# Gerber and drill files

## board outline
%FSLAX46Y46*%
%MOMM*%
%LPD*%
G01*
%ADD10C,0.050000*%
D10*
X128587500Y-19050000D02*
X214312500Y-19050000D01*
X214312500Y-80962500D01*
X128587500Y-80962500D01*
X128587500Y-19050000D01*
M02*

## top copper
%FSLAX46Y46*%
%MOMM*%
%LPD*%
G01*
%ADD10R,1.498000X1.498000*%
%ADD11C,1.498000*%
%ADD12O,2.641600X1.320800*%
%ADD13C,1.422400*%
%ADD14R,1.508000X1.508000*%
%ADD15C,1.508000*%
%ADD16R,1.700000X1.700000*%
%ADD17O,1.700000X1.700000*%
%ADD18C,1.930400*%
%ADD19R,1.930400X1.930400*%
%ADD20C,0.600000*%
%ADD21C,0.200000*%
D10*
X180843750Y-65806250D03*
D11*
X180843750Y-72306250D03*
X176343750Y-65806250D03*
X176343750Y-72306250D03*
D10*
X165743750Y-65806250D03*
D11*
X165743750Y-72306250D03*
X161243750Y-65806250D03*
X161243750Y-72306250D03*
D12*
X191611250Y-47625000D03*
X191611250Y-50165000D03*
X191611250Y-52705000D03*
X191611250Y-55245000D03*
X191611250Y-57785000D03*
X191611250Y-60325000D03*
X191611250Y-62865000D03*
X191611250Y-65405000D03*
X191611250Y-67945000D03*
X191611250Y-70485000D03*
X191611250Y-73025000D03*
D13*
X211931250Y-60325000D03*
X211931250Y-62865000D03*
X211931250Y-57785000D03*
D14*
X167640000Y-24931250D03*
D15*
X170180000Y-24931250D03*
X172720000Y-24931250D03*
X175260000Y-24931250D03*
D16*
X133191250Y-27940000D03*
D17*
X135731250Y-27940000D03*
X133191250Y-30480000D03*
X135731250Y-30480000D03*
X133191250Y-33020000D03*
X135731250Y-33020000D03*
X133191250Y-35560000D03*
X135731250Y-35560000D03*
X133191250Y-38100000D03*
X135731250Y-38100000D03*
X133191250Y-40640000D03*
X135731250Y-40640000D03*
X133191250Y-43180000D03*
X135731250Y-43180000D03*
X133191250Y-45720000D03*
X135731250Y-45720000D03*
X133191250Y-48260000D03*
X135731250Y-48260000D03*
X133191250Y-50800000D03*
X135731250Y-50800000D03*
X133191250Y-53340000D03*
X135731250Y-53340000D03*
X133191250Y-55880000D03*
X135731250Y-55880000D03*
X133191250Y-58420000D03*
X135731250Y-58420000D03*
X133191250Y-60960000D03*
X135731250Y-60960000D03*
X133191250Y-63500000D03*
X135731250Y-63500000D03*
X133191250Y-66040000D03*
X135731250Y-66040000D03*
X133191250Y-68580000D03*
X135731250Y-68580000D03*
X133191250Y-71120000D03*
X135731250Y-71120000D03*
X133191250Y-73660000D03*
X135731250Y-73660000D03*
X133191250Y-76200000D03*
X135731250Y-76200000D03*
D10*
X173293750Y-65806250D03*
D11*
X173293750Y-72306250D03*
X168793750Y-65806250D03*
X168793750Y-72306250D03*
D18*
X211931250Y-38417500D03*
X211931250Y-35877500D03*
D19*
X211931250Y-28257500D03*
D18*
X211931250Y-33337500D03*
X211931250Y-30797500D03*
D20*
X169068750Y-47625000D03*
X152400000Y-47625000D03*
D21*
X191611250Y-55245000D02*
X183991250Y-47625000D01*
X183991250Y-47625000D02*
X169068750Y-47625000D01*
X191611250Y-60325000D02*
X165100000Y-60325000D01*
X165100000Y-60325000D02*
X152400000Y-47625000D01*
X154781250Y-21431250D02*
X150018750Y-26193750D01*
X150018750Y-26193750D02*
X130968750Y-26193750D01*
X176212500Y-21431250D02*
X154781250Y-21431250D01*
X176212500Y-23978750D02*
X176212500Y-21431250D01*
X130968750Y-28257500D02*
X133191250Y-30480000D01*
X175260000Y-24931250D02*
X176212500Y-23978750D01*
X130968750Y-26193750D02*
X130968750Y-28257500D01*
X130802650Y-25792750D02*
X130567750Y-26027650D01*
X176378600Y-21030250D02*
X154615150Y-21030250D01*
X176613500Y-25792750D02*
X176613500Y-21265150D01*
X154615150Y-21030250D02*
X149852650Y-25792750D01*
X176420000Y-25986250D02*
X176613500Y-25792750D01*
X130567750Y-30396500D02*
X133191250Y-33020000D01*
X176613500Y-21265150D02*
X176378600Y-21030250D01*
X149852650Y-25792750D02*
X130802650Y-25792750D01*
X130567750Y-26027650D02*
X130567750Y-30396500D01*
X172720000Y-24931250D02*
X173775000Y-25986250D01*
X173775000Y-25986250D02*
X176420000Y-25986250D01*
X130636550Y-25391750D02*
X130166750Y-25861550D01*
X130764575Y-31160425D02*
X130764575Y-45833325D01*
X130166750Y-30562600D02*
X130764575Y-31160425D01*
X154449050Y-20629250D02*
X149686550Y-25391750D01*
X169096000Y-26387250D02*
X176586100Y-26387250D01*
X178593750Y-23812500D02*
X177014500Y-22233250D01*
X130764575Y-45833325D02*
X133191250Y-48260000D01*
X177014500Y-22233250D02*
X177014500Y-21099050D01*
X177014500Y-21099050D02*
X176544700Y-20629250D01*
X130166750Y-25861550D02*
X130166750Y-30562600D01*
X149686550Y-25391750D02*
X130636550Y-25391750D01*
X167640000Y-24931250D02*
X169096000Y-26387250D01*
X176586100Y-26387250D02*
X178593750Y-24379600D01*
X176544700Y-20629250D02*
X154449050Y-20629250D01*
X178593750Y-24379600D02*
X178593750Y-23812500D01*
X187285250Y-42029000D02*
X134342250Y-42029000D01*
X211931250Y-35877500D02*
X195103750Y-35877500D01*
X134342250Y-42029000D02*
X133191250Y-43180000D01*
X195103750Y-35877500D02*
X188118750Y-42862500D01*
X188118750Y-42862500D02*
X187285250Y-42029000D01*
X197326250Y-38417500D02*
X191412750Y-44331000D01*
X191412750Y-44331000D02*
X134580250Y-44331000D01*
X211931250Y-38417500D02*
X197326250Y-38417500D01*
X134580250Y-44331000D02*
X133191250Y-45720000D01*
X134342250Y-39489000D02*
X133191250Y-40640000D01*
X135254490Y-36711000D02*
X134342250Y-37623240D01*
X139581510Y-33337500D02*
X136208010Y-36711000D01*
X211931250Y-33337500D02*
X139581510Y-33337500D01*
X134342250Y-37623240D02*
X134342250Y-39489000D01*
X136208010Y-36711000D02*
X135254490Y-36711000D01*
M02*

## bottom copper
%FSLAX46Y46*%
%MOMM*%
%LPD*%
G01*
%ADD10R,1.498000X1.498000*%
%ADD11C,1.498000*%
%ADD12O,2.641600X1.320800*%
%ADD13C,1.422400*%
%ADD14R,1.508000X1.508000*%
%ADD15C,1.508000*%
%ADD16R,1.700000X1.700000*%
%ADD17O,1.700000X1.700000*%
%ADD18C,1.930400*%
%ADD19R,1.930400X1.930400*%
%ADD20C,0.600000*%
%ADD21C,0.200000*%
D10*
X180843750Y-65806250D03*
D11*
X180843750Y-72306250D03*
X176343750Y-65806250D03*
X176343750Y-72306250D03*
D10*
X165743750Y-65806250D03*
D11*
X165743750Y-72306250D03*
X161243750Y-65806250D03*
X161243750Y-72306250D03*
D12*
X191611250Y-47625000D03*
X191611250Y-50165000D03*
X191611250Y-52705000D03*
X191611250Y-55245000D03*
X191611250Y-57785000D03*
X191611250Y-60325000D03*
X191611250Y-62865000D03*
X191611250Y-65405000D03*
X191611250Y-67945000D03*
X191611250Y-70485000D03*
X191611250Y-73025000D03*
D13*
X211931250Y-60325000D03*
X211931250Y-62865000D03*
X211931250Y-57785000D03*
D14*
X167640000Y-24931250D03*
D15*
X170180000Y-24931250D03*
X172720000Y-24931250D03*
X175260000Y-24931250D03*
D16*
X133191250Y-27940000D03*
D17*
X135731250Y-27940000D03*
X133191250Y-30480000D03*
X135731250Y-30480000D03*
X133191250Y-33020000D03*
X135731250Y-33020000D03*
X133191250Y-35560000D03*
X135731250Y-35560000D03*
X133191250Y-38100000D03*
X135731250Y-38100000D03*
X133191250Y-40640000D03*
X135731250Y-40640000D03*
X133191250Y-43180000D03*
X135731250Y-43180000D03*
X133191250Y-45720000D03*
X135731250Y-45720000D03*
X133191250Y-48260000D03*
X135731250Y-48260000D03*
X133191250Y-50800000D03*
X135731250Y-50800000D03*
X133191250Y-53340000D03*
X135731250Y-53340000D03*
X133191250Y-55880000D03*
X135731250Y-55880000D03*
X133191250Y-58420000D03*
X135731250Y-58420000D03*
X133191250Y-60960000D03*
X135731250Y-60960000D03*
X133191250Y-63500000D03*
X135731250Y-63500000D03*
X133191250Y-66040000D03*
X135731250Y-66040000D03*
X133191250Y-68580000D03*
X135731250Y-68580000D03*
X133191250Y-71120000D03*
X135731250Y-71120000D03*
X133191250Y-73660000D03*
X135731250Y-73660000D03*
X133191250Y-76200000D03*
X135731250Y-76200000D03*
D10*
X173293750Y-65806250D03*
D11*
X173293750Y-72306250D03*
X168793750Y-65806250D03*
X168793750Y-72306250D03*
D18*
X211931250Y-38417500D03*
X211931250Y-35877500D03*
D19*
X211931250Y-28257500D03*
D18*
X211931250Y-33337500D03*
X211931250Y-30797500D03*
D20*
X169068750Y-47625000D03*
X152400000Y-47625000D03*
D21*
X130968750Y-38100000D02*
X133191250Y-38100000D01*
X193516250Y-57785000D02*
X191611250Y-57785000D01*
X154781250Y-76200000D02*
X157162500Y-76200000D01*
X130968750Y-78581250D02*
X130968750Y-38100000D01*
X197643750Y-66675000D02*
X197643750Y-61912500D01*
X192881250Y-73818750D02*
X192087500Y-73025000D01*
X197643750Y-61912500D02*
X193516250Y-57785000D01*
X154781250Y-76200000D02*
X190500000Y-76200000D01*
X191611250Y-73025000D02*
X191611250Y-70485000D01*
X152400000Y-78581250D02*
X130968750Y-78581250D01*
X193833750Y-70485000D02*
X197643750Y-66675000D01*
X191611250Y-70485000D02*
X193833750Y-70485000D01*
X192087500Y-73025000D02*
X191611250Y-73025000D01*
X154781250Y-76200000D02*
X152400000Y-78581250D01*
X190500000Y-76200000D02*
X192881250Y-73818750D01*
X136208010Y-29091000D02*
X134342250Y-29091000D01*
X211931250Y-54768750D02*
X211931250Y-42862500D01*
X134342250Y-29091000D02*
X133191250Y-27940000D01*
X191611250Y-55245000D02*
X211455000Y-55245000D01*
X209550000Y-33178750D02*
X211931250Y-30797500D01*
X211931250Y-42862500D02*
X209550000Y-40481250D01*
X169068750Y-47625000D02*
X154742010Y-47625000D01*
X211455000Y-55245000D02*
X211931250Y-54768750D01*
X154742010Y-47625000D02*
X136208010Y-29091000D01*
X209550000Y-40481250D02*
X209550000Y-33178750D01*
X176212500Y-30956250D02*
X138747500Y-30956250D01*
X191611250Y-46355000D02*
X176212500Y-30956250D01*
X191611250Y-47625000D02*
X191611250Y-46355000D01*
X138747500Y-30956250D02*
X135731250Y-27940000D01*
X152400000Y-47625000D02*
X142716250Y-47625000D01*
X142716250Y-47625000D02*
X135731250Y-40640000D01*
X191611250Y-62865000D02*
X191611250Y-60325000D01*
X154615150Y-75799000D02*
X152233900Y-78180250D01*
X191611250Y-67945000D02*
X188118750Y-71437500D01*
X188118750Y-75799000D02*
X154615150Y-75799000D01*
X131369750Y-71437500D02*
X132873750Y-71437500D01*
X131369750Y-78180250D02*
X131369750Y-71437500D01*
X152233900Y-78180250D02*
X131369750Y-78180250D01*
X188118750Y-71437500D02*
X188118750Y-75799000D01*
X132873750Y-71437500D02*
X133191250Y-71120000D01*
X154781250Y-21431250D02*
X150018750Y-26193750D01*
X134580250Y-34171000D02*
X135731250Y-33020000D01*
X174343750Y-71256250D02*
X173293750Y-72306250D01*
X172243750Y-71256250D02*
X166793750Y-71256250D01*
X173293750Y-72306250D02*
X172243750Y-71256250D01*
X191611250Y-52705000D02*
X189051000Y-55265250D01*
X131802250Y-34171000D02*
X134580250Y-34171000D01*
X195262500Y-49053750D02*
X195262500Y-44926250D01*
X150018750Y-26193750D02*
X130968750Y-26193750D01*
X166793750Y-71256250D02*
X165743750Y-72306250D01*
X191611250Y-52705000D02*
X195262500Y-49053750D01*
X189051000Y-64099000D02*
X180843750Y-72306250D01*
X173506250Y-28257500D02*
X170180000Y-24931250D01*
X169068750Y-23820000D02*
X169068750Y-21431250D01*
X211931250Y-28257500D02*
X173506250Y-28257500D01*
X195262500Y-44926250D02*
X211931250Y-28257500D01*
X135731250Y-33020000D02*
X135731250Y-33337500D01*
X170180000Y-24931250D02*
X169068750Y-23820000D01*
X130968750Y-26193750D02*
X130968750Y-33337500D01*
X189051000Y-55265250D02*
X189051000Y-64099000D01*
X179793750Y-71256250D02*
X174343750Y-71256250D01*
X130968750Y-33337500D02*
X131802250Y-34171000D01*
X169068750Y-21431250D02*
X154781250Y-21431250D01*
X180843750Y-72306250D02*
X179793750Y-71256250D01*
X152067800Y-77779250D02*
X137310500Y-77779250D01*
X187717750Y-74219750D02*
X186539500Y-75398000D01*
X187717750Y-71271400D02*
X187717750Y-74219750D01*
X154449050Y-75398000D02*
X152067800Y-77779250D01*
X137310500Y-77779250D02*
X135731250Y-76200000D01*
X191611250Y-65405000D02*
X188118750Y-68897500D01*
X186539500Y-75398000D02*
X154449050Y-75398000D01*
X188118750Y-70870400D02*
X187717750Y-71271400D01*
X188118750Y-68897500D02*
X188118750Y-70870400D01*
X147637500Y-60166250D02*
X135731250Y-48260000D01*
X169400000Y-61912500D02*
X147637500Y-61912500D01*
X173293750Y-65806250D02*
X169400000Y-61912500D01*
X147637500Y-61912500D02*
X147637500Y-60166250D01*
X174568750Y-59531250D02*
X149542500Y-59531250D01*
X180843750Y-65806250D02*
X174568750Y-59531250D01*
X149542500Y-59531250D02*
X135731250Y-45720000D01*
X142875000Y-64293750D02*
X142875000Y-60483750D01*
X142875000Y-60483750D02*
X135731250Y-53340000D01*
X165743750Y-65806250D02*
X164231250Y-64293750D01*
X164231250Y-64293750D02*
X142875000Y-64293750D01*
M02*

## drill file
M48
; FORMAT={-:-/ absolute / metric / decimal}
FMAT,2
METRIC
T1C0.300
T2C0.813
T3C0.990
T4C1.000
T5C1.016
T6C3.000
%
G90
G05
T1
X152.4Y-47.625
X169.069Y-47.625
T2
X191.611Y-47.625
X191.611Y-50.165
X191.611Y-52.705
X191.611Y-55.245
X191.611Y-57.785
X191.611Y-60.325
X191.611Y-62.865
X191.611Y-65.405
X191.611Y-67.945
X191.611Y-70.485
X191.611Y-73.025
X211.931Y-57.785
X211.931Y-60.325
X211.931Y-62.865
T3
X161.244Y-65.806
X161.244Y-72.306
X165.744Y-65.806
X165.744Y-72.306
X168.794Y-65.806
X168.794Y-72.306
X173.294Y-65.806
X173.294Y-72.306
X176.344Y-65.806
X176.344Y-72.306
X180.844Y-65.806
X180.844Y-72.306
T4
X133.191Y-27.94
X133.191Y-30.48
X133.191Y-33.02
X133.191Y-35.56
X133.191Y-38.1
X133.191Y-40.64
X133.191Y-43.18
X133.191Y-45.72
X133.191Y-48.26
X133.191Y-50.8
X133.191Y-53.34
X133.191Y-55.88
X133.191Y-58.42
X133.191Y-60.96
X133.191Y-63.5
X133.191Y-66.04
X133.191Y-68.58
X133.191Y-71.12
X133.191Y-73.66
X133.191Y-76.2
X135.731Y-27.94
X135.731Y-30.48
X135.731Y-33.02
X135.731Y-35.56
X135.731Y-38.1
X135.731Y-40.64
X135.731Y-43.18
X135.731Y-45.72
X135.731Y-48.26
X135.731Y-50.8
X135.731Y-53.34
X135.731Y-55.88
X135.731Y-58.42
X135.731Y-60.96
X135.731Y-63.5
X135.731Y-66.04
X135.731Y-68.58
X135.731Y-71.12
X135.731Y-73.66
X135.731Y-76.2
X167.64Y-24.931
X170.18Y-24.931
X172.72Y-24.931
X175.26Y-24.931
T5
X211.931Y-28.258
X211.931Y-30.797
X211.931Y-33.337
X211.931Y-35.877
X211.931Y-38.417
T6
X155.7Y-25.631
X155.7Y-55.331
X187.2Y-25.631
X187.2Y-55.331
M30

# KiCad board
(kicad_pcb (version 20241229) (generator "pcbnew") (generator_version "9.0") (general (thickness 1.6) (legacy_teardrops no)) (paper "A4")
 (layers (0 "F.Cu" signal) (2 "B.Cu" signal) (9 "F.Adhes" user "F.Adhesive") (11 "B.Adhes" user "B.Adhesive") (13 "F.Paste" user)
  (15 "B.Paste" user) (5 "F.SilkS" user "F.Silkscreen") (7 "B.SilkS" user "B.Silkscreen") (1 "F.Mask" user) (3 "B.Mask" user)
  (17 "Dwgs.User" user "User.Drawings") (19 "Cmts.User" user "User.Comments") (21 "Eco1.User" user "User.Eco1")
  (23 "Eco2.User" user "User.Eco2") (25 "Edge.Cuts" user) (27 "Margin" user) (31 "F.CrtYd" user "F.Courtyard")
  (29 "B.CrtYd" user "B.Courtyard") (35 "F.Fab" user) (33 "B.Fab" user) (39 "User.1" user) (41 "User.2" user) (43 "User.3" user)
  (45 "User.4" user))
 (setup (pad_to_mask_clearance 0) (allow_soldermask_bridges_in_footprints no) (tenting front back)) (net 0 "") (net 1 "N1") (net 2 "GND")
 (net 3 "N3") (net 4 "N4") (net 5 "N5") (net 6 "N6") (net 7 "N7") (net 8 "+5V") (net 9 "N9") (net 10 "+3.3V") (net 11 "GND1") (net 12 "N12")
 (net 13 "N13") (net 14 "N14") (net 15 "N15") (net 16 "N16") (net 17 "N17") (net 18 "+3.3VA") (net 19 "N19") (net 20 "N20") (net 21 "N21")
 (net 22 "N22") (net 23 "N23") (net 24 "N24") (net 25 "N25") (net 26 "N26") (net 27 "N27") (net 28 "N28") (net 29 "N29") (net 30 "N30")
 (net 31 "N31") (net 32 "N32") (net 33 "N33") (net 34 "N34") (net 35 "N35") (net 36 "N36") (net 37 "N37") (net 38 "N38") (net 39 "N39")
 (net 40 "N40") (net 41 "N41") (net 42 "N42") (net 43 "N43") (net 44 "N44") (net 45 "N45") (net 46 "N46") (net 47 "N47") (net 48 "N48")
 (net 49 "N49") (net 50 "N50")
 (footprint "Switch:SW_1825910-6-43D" (layer "F.Cu") (at 178.59375 69.05625 -90)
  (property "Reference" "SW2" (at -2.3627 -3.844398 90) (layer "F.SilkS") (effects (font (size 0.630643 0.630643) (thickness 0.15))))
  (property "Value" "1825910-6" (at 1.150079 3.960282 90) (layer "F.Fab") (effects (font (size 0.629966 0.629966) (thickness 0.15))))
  (pad "1" thru_hole rect (at -3.25 -2.25 270) (size 1.498 1.498) (drill 0.99) (layers "*.Cu" "*.Mask") (remove_unused_layers no)
   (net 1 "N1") (solder_mask_margin 0.102))
  (pad "2" thru_hole circle (at 3.25 -2.25 270) (size 1.498 1.498) (drill 0.99) (layers "*.Cu" "*.Mask") (remove_unused_layers no)
   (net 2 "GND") (solder_mask_margin 0.102))
  (pad "3" thru_hole circle (at -3.25 2.25 270) (size 1.498 1.498) (drill 0.99) (layers "*.Cu" "*.Mask") (remove_unused_layers no)
   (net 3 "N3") (solder_mask_margin 0.102))
  (pad "4" thru_hole circle (at 3.25 2.25 270) (size 1.498 1.498) (drill 0.99) (layers "*.Cu" "*.Mask") (remove_unused_layers no)
   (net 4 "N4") (solder_mask_margin 0.102)))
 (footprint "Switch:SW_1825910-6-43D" (layer "F.Cu") (at 163.49375 69.05625 -90)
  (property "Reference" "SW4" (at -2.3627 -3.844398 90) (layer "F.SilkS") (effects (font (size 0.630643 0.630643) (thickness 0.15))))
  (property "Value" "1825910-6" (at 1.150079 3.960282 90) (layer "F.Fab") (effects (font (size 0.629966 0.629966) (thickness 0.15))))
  (pad "1" thru_hole rect (at -3.25 -2.25 270) (size 1.498 1.498) (drill 0.99) (layers "*.Cu" "*.Mask") (remove_unused_layers no)
   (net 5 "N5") (solder_mask_margin 0.102))
  (pad "2" thru_hole circle (at 3.25 -2.25 270) (size 1.498 1.498) (drill 0.99) (layers "*.Cu" "*.Mask") (remove_unused_layers no)
   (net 2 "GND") (solder_mask_margin 0.102))
  (pad "3" thru_hole circle (at -3.25 2.25 270) (size 1.498 1.498) (drill 0.99) (layers "*.Cu" "*.Mask") (remove_unused_layers no)
   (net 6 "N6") (solder_mask_margin 0.102))
  (pad "4" thru_hole circle (at 3.25 2.25 270) (size 1.498 1.498) (drill 0.99) (layers "*.Cu" "*.Mask") (remove_unused_layers no)
   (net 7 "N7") (solder_mask_margin 0.102)))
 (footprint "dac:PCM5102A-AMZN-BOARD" (layer "F.Cu") (at 191.61125 47.625 -90)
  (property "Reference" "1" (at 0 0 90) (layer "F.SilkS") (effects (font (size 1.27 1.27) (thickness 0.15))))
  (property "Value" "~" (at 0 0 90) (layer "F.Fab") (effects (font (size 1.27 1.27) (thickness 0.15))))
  (pad "1" thru_hole oval (at 0 0) (size 2.6416 1.3208) (drill 0.8128) (layers "*.Cu" "*.Mask") (remove_unused_layers no) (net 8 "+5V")
   (solder_mask_margin 0.1016) (thermal_bridge_angle 0))
  (pad "2" thru_hole oval (at 2.54 0) (size 2.6416 1.3208) (drill 0.8128) (layers "*.Cu" "*.Mask") (remove_unused_layers no) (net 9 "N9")
   (solder_mask_margin 0.1016) (thermal_bridge_angle 0))
  (pad "3" thru_hole oval (at 5.08 0) (size 2.6416 1.3208) (drill 0.8128) (layers "*.Cu" "*.Mask") (remove_unused_layers no) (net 2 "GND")
   (solder_mask_margin 0.1016) (thermal_bridge_angle 0))
  (pad "4" thru_hole oval (at 7.62 0) (size 2.6416 1.3208) (drill 0.8128) (layers "*.Cu" "*.Mask") (remove_unused_layers no)
   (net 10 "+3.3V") (solder_mask_margin 0.1016) (thermal_bridge_angle 0))
  (pad "5" thru_hole oval (at 10.16 0) (size 2.6416 1.3208) (drill 0.8128) (layers "*.Cu" "*.Mask") (remove_unused_layers no)
   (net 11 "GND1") (solder_mask_margin 0.1016) (thermal_bridge_angle 0))
  (pad "6" thru_hole oval (at 12.7 0) (size 2.6416 1.3208) (drill 0.8128) (layers "*.Cu" "*.Mask") (remove_unused_layers no) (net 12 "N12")
   (solder_mask_margin 0.1016) (thermal_bridge_angle 0))
  (pad "7" thru_hole oval (at 15.24 0) (size 2.6416 1.3208) (drill 0.8128) (layers "*.Cu" "*.Mask") (remove_unused_layers no) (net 12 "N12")
   (solder_mask_margin 0.1016) (thermal_bridge_angle 0))
  (pad "8" thru_hole oval (at 17.78 0) (size 2.6416 1.3208) (drill 0.8128) (layers "*.Cu" "*.Mask") (remove_unused_layers no) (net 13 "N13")
   (solder_mask_margin 0.1016) (thermal_bridge_angle 0))
  (pad "9" thru_hole oval (at 20.32 0) (size 2.6416 1.3208) (drill 0.8128) (layers "*.Cu" "*.Mask") (remove_unused_layers no) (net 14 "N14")
   (solder_mask_margin 0.1016) (thermal_bridge_angle 0))
  (pad "10" thru_hole oval (at 22.86 0) (size 2.6416 1.3208) (drill 0.8128) (layers "*.Cu" "*.Mask") (remove_unused_layers no)
   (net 11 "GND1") (solder_mask_margin 0.1016) (thermal_bridge_angle 0))
  (pad "11" thru_hole oval (at 25.4 0) (size 2.6416 1.3208) (drill 0.8128) (layers "*.Cu" "*.Mask") (remove_unused_layers no)
   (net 11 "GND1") (solder_mask_margin 0.1016) (thermal_bridge_angle 0))
  (pad "G" thru_hole circle (at 12.7 -20.32 270) (size 1.4224 1.4224) (drill 0.8128) (layers "*.Cu" "*.Mask") (remove_unused_layers no)
   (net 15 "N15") (solder_mask_margin 0.1016) (thermal_bridge_angle 0))
  (pad "L" thru_hole circle (at 15.24 -20.32 270) (size 1.4224 1.4224) (drill 0.8128) (layers "*.Cu" "*.Mask") (remove_unused_layers no)
   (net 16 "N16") (solder_mask_margin 0.1016) (thermal_bridge_angle 0))
  (pad "R" thru_hole circle (at 10.16 -20.32 270) (size 1.4224 1.4224) (drill 0.8128) (layers "*.Cu" "*.Mask") (remove_unused_layers no)
   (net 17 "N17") (solder_mask_margin 0.1016) (thermal_bridge_angle 0)))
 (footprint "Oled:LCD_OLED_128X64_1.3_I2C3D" (layer "F.Cu") (at 171.45 40.48125)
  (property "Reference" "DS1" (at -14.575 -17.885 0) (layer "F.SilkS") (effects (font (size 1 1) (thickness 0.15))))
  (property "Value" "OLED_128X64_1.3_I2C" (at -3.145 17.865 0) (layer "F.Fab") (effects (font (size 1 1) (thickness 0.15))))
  (pad "" np_thru_hole circle (at -15.75 -14.85) (size 3 3) (drill 3) (layers "*.Cu" "*.Mask"))
  (pad "" np_thru_hole circle (at -15.75 14.85) (size 3 3) (drill 3) (layers "*.Cu" "*.Mask"))
  (pad "" np_thru_hole circle (at 15.75 -14.85) (size 3 3) (drill 3) (layers "*.Cu" "*.Mask"))
  (pad "" np_thru_hole circle (at 15.75 14.85) (size 3 3) (drill 3) (layers "*.Cu" "*.Mask"))
  (pad "1" thru_hole rect (at -3.81 -15.55) (size 1.508 1.508) (drill 1) (layers "*.Cu" "*.Mask") (remove_unused_layers no)
   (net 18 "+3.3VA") (solder_mask_margin 0.102))
  (pad "2" thru_hole circle (at -1.27 -15.55) (size 1.508 1.508) (drill 1) (layers "*.Cu" "*.Mask") (remove_unused_layers no) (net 2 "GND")
   (solder_mask_margin 0.102))
  (pad "3" thru_hole circle (at 1.27 -15.55) (size 1.508 1.508) (drill 1) (layers "*.Cu" "*.Mask") (remove_unused_layers no) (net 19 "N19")
   (solder_mask_margin 0.102))
  (pad "4" thru_hole circle (at 3.81 -15.55) (size 1.508 1.508) (drill 1) (layers "*.Cu" "*.Mask") (remove_unused_layers no) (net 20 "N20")
   (solder_mask_margin 0.102)))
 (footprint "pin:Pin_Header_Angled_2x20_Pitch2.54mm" (layer "F.Cu") (at 133.19125 27.94)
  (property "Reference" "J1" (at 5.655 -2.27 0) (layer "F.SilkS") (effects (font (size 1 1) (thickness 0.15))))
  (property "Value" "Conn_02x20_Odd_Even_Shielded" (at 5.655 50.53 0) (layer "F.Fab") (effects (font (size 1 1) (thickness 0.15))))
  (pad "1" thru_hole rect (at 0 0) (size 1.7 1.7) (drill 1) (layers "*.Cu" "*.Mask") (remove_unused_layers no) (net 10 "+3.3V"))
  (pad "2" thru_hole oval (at 2.54 0) (size 1.7 1.7) (drill 1) (layers "*.Cu" "*.Mask") (remove_unused_layers no) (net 8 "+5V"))
  (pad "3" thru_hole oval (at 0 2.54) (size 1.7 1.7) (drill 1) (layers "*.Cu" "*.Mask") (remove_unused_layers no) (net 20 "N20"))
  (pad "4" thru_hole oval (at 2.54 2.54) (size 1.7 1.7) (drill 1) (layers "*.Cu" "*.Mask") (remove_unused_layers no) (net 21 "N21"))
  (pad "5" thru_hole oval (at 0 5.08) (size 1.7 1.7) (drill 1) (layers "*.Cu" "*.Mask") (remove_unused_layers no) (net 19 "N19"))
  (pad "6" thru_hole oval (at 2.54 5.08) (size 1.7 1.7) (drill 1) (layers "*.Cu" "*.Mask") (remove_unused_layers no) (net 2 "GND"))
  (pad "7" thru_hole oval (at 0 7.62) (size 1.7 1.7) (drill 1) (layers "*.Cu" "*.Mask") (remove_unused_layers no) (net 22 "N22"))
  (pad "8" thru_hole oval (at 2.54 7.62) (size 1.7 1.7) (drill 1) (layers "*.Cu" "*.Mask") (remove_unused_layers no) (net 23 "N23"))
  (pad "9" thru_hole oval (at 0 10.16) (size 1.7 1.7) (drill 1) (layers "*.Cu" "*.Mask") (remove_unused_layers no) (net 11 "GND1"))
  (pad "10" thru_hole oval (at 2.54 10.16) (size 1.7 1.7) (drill 1) (layers "*.Cu" "*.Mask") (remove_unused_layers no) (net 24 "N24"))
  (pad "11" thru_hole oval (at 0 12.7) (size 1.7 1.7) (drill 1) (layers "*.Cu" "*.Mask") (remove_unused_layers no) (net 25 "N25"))
  (pad "12" thru_hole oval (at 2.54 12.7) (size 1.7 1.7) (drill 1) (layers "*.Cu" "*.Mask") (remove_unused_layers no) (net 12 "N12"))
  (pad "13" thru_hole oval (at 0 15.24) (size 1.7 1.7) (drill 1) (layers "*.Cu" "*.Mask") (remove_unused_layers no) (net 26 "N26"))
  (pad "14" thru_hole oval (at 2.54 15.24) (size 1.7 1.7) (drill 1) (layers "*.Cu" "*.Mask") (remove_unused_layers no) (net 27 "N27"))
  (pad "15" thru_hole oval (at 0 17.78) (size 1.7 1.7) (drill 1) (layers "*.Cu" "*.Mask") (remove_unused_layers no) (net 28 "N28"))
  (pad "16" thru_hole oval (at 2.54 17.78) (size 1.7 1.7) (drill 1) (layers "*.Cu" "*.Mask") (remove_unused_layers no) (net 1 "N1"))
  (pad "17" thru_hole oval (at 0 20.32) (size 1.7 1.7) (drill 1) (layers "*.Cu" "*.Mask") (remove_unused_layers no) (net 18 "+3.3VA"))
  (pad "18" thru_hole oval (at 2.54 20.32) (size 1.7 1.7) (drill 1) (layers "*.Cu" "*.Mask") (remove_unused_layers no) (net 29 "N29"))
  (pad "19" thru_hole oval (at 0 22.86) (size 1.7 1.7) (drill 1) (layers "*.Cu" "*.Mask") (remove_unused_layers no) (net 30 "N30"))
  (pad "20" thru_hole oval (at 2.54 22.86) (size 1.7 1.7) (drill 1) (layers "*.Cu" "*.Mask") (remove_unused_layers no) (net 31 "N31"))
  (pad "21" thru_hole oval (at 0 25.4) (size 1.7 1.7) (drill 1) (layers "*.Cu" "*.Mask") (remove_unused_layers no) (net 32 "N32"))
  (pad "22" thru_hole oval (at 2.54 25.4) (size 1.7 1.7) (drill 1) (layers "*.Cu" "*.Mask") (remove_unused_layers no) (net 5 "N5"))
  (pad "23" thru_hole oval (at 0 27.94) (size 1.7 1.7) (drill 1) (layers "*.Cu" "*.Mask") (remove_unused_layers no) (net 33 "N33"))
  (pad "24" thru_hole oval (at 2.54 27.94) (size 1.7 1.7) (drill 1) (layers "*.Cu" "*.Mask") (remove_unused_layers no) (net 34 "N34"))
  (pad "25" thru_hole oval (at 0 30.48) (size 1.7 1.7) (drill 1) (layers "*.Cu" "*.Mask") (remove_unused_layers no) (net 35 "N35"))
  (pad "26" thru_hole oval (at 2.54 30.48) (size 1.7 1.7) (drill 1) (layers "*.Cu" "*.Mask") (remove_unused_layers no) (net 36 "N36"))
  (pad "27" thru_hole oval (at 0 33.02) (size 1.7 1.7) (drill 1) (layers "*.Cu" "*.Mask") (remove_unused_layers no) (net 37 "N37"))
  (pad "28" thru_hole oval (at 2.54 33.02) (size 1.7 1.7) (drill 1) (layers "*.Cu" "*.Mask") (remove_unused_layers no) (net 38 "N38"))
  (pad "29" thru_hole oval (at 0 35.56) (size 1.7 1.7) (drill 1) (layers "*.Cu" "*.Mask") (remove_unused_layers no) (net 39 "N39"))
  (pad "30" thru_hole oval (at 2.54 35.56) (size 1.7 1.7) (drill 1) (layers "*.Cu" "*.Mask") (remove_unused_layers no) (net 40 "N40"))
  (pad "31" thru_hole oval (at 0 38.1) (size 1.7 1.7) (drill 1) (layers "*.Cu" "*.Mask") (remove_unused_layers no) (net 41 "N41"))
  (pad "32" thru_hole oval (at 2.54 38.1) (size 1.7 1.7) (drill 1) (layers "*.Cu" "*.Mask") (remove_unused_layers no) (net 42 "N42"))
  (pad "33" thru_hole oval (at 0 40.64) (size 1.7 1.7) (drill 1) (layers "*.Cu" "*.Mask") (remove_unused_layers no) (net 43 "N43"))
  (pad "34" thru_hole oval (at 2.54 40.64) (size 1.7 1.7) (drill 1) (layers "*.Cu" "*.Mask") (remove_unused_layers no) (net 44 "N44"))
  (pad "35" thru_hole oval (at 0 43.18) (size 1.7 1.7) (drill 1) (layers "*.Cu" "*.Mask") (remove_unused_layers no) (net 14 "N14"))
  (pad "36" thru_hole oval (at 2.54 43.18) (size 1.7 1.7) (drill 1) (layers "*.Cu" "*.Mask") (remove_unused_layers no) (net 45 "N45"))
  (pad "37" thru_hole oval (at 0 45.72) (size 1.7 1.7) (drill 1) (layers "*.Cu" "*.Mask") (remove_unused_layers no) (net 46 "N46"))
  (pad "38" thru_hole oval (at 2.54 45.72) (size 1.7 1.7) (drill 1) (layers "*.Cu" "*.Mask") (remove_unused_layers no) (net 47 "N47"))
  (pad "39" thru_hole oval (at 0 48.26) (size 1.7 1.7) (drill 1) (layers "*.Cu" "*.Mask") (remove_unused_layers no) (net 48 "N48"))
  (pad "40" thru_hole oval (at 2.54 48.26) (size 1.7 1.7) (drill 1) (layers "*.Cu" "*.Mask") (remove_unused_layers no) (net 13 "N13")))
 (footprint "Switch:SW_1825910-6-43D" (layer "F.Cu") (at 171.04375 69.05625 -90)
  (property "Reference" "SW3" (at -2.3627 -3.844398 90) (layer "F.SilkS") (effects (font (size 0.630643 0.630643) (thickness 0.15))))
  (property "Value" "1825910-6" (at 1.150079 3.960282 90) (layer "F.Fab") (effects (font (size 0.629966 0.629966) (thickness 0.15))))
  (pad "1" thru_hole rect (at -3.25 -2.25 270) (size 1.498 1.498) (drill 0.99) (layers "*.Cu" "*.Mask") (remove_unused_layers no)
   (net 29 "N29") (solder_mask_margin 0.102))
  (pad "2" thru_hole circle (at 3.25 -2.25 270) (size 1.498 1.498) (drill 0.99) (layers "*.Cu" "*.Mask") (remove_unused_layers no)
   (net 2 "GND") (solder_mask_margin 0.102))
  (pad "3" thru_hole circle (at -3.25 2.25 270) (size 1.498 1.498) (drill 0.99) (layers "*.Cu" "*.Mask") (remove_unused_layers no)
   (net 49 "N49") (solder_mask_margin 0.102))
  (pad "4" thru_hole circle (at 3.25 2.25 270) (size 1.498 1.498) (drill 0.99) (layers "*.Cu" "*.Mask") (remove_unused_layers no)
   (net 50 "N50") (solder_mask_margin 0.102)))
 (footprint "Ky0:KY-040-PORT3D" (layer "B.Cu") (at 211.93125 32.0675 90)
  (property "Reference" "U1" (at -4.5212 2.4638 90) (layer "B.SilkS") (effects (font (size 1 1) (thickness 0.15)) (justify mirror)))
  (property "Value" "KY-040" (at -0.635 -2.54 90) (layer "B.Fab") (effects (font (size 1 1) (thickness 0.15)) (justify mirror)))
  (pad "CLK" thru_hole circle (at -6.35 0 90) (size 1.9304 1.9304) (drill 1.016) (layers "*.Cu" "*.Mask") (remove_unused_layers no)
   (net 28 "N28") (solder_mask_margin 0.102))
  (pad "DT" thru_hole circle (at -3.81 0 90) (size 1.9304 1.9304) (drill 1.016) (layers "*.Cu" "*.Mask") (remove_unused_layers no)
   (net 26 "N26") (solder_mask_margin 0.102))
  (pad "GND" thru_hole rect (at 3.81 0 90) (size 1.9304 1.9304) (drill 1.016) (layers "*.Cu" "*.Mask") (remove_unused_layers no)
   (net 2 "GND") (solder_mask_margin 0.102))
  (pad "SW" thru_hole circle (at -1.27 0 90) (size 1.9304 1.9304) (drill 1.016) (layers "*.Cu" "*.Mask") (remove_unused_layers no)
   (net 25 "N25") (solder_mask_margin 0.102))
  (pad "VCC" thru_hole circle (at 1.27 0 90) (size 1.9304 1.9304) (drill 1.016) (layers "*.Cu" "*.Mask") (remove_unused_layers no)
   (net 10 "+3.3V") (solder_mask_margin 0.102)))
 (gr_rect (start 128.5875 19.05) (end 214.3125 80.9625) (stroke (width 0.05) (type default)) (fill no) (layer "Edge.Cuts"))
 (segment (start 130.96875 38.1) (end 133.19125 38.1) (width 0.2) (layer "B.Cu") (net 11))
 (segment (start 193.51625 57.785) (end 191.61125 57.785) (width 0.2) (layer "B.Cu") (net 11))
 (segment (start 154.78125 76.2) (end 157.1625 76.2) (width 0.2) (layer "B.Cu") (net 11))
 (segment (start 130.96875 78.58125) (end 130.96875 38.1) (width 0.2) (layer "B.Cu") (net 11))
 (segment (start 197.64375 66.675) (end 197.64375 61.9125) (width 0.2) (layer "B.Cu") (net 11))
 (segment (start 192.88125 73.81875) (end 192.0875 73.025) (width 0.2) (layer "B.Cu") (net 11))
 (segment (start 197.64375 61.9125) (end 193.51625 57.785) (width 0.2) (layer "B.Cu") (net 11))
 (segment (start 154.78125 76.2) (end 190.5 76.2) (width 0.2) (layer "B.Cu") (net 11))
 (segment (start 191.61125 73.025) (end 191.61125 70.485) (width 0.2) (layer "B.Cu") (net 11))
 (segment (start 152.4 78.58125) (end 130.96875 78.58125) (width 0.2) (layer "B.Cu") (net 11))
 (segment (start 193.83375 70.485) (end 197.64375 66.675) (width 0.2) (layer "B.Cu") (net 11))
 (segment (start 191.61125 70.485) (end 193.83375 70.485) (width 0.2) (layer "B.Cu") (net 11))
 (segment (start 192.0875 73.025) (end 191.61125 73.025) (width 0.2) (layer "B.Cu") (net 11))
 (segment (start 154.78125 76.2) (end 152.4 78.58125) (width 0.2) (layer "B.Cu") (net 11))
 (segment (start 190.5 76.2) (end 192.88125 73.81875) (width 0.2) (layer "B.Cu") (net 11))
 (segment (start 191.61125 55.245) (end 183.99125 47.625) (width 0.2) (layer "F.Cu") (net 10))
 (segment (start 183.99125 47.625) (end 169.06875 47.625) (width 0.2) (layer "F.Cu") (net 10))
 (via (at 169.06875 47.625) (size 0.6) (drill 0.3) (layers "F.Cu" "B.Cu") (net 10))
 (segment (start 136.20801 29.091) (end 134.34225 29.091) (width 0.2) (layer "B.Cu") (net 10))
 (segment (start 211.93125 54.76875) (end 211.93125 42.8625) (width 0.2) (layer "B.Cu") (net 10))
 (segment (start 134.34225 29.091) (end 133.19125 27.94) (width 0.2) (layer "B.Cu") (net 10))
 (segment (start 191.61125 55.245) (end 211.455 55.245) (width 0.2) (layer "B.Cu") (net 10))
 (segment (start 209.55 33.17875) (end 211.93125 30.7975) (width 0.2) (layer "B.Cu") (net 10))
 (segment (start 211.93125 42.8625) (end 209.55 40.48125) (width 0.2) (layer "B.Cu") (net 10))
 (segment (start 169.06875 47.625) (end 154.74201 47.625) (width 0.2) (layer "B.Cu") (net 10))
 (segment (start 211.455 55.245) (end 211.93125 54.76875) (width 0.2) (layer "B.Cu") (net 10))
 (segment (start 154.74201 47.625) (end 136.20801 29.091) (width 0.2) (layer "B.Cu") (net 10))
 (segment (start 209.55 40.48125) (end 209.55 33.17875) (width 0.2) (layer "B.Cu") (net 10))
 (segment (start 176.2125 30.95625) (end 138.7475 30.95625) (width 0.2) (layer "B.Cu") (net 8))
 (segment (start 191.61125 46.355) (end 176.2125 30.95625) (width 0.2) (layer "B.Cu") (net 8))
 (segment (start 191.61125 47.625) (end 191.61125 46.355) (width 0.2) (layer "B.Cu") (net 8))
 (segment (start 138.7475 30.95625) (end 135.73125 27.94) (width 0.2) (layer "B.Cu") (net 8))
 (segment (start 191.61125 60.325) (end 165.1 60.325) (width 0.2) (layer "F.Cu") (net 12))
 (segment (start 165.1 60.325) (end 152.4 47.625) (width 0.2) (layer "F.Cu") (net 12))
 (via (at 152.4 47.625) (size 0.6) (drill 0.3) (layers "F.Cu" "B.Cu") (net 12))
 (segment (start 152.4 47.625) (end 142.71625 47.625) (width 0.2) (layer "B.Cu") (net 12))
 (segment (start 142.71625 47.625) (end 135.73125 40.64) (width 0.2) (layer "B.Cu") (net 12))
 (segment (start 191.61125 62.865) (end 191.61125 60.325) (width 0.2) (layer "B.Cu") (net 12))
 (segment (start 154.61515 75.799) (end 152.2339 78.18025) (width 0.2) (layer "B.Cu") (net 14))
 (segment (start 191.61125 67.945) (end 188.11875 71.4375) (width 0.2) (layer "B.Cu") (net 14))
 (segment (start 188.11875 75.799) (end 154.61515 75.799) (width 0.2) (layer "B.Cu") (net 14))
 (segment (start 131.36975 71.4375) (end 132.87375 71.4375) (width 0.2) (layer "B.Cu") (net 14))
 (segment (start 131.36975 78.18025) (end 131.36975 71.4375) (width 0.2) (layer "B.Cu") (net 14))
 (segment (start 152.2339 78.18025) (end 131.36975 78.18025) (width 0.2) (layer "B.Cu") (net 14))
 (segment (start 188.11875 71.4375) (end 188.11875 75.799) (width 0.2) (layer "B.Cu") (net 14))
 (segment (start 132.87375 71.4375) (end 133.19125 71.12) (width 0.2) (layer "B.Cu") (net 14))
 (segment (start 154.78125 21.43125) (end 150.01875 26.19375) (width 0.2) (layer "B.Cu") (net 2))
 (segment (start 134.58025 34.171) (end 135.73125 33.02) (width 0.2) (layer "B.Cu") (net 2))
 (segment (start 174.34375 71.25625) (end 173.29375 72.30625) (width 0.2) (layer "B.Cu") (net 2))
 (segment (start 172.24375 71.25625) (end 166.79375 71.25625) (width 0.2) (layer "B.Cu") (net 2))
 (segment (start 173.29375 72.30625) (end 172.24375 71.25625) (width 0.2) (layer "B.Cu") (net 2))
 (segment (start 191.61125 52.705) (end 189.051 55.26525) (width 0.2) (layer "B.Cu") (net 2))
 (segment (start 131.80225 34.171) (end 134.58025 34.171) (width 0.2) (layer "B.Cu") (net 2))
 (segment (start 195.2625 49.05375) (end 195.2625 44.92625) (width 0.2) (layer "B.Cu") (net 2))
 (segment (start 150.01875 26.19375) (end 130.96875 26.19375) (width 0.2) (layer "B.Cu") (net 2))
 (segment (start 166.79375 71.25625) (end 165.74375 72.30625) (width 0.2) (layer "B.Cu") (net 2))
 (segment (start 191.61125 52.705) (end 195.2625 49.05375) (width 0.2) (layer "B.Cu") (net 2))
 (segment (start 189.051 64.099) (end 180.84375 72.30625) (width 0.2) (layer "B.Cu") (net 2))
 (segment (start 173.50625 28.2575) (end 170.18 24.93125) (width 0.2) (layer "B.Cu") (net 2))
 (segment (start 169.06875 23.82) (end 169.06875 21.43125) (width 0.2) (layer "B.Cu") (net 2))
 (segment (start 211.93125 28.2575) (end 173.50625 28.2575) (width 0.2) (layer "B.Cu") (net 2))
 (segment (start 195.2625 44.92625) (end 211.93125 28.2575) (width 0.2) (layer "B.Cu") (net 2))
 (segment (start 135.73125 33.02) (end 135.73125 33.3375) (width 0.2) (layer "B.Cu") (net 2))
 (segment (start 170.18 24.93125) (end 169.06875 23.82) (width 0.2) (layer "B.Cu") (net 2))
 (segment (start 130.96875 26.19375) (end 130.96875 33.3375) (width 0.2) (layer "B.Cu") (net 2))
 (segment (start 189.051 55.26525) (end 189.051 64.099) (width 0.2) (layer "B.Cu") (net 2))
 (segment (start 179.79375 71.25625) (end 174.34375 71.25625) (width 0.2) (layer "B.Cu") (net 2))
 (segment (start 130.96875 33.3375) (end 131.80225 34.171) (width 0.2) (layer "B.Cu") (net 2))
 (segment (start 169.06875 21.43125) (end 154.78125 21.43125) (width 0.2) (layer "B.Cu") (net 2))
 (segment (start 180.84375 72.30625) (end 179.79375 71.25625) (width 0.2) (layer "B.Cu") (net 2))
 (segment (start 152.0678 77.77925) (end 137.3105 77.77925) (width 0.2) (layer "B.Cu") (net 13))
 (segment (start 187.71775 74.21975) (end 186.5395 75.398) (width 0.2) (layer "B.Cu") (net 13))
 (segment (start 187.71775 71.2714) (end 187.71775 74.21975) (width 0.2) (layer "B.Cu") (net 13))
 (segment (start 154.44905 75.398) (end 152.0678 77.77925) (width 0.2) (layer "B.Cu") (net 13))
 (segment (start 137.3105 77.77925) (end 135.73125 76.2) (width 0.2) (layer "B.Cu") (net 13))
 (segment (start 191.61125 65.405) (end 188.11875 68.8975) (width 0.2) (layer "B.Cu") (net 13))
 (segment (start 186.5395 75.398) (end 154.44905 75.398) (width 0.2) (layer "B.Cu") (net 13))
 (segment (start 188.11875 70.8704) (end 187.71775 71.2714) (width 0.2) (layer "B.Cu") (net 13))
 (segment (start 188.11875 68.8975) (end 188.11875 70.8704) (width 0.2) (layer "B.Cu") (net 13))
 (segment (start 154.78125 21.43125) (end 150.01875 26.19375) (width 0.2) (layer "F.Cu") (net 20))
 (segment (start 150.01875 26.19375) (end 130.96875 26.19375) (width 0.2) (layer "F.Cu") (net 20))
 (segment (start 176.2125 21.43125) (end 154.78125 21.43125) (width 0.2) (layer "F.Cu") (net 20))
 (segment (start 176.2125 23.97875) (end 176.2125 21.43125) (width 0.2) (layer "F.Cu") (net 20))
 (segment (start 130.96875 28.2575) (end 133.19125 30.48) (width 0.2) (layer "F.Cu") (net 20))
 (segment (start 175.26 24.93125) (end 176.2125 23.97875) (width 0.2) (layer "F.Cu") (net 20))
 (segment (start 130.96875 26.19375) (end 130.96875 28.2575) (width 0.2) (layer "F.Cu") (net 20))
 (segment (start 130.80265 25.79275) (end 130.56775 26.02765) (width 0.2) (layer "F.Cu") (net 19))
 (segment (start 176.3786 21.03025) (end 154.61515 21.03025) (width 0.2) (layer "F.Cu") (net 19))
 (segment (start 176.6135 25.79275) (end 176.6135 21.26515) (width 0.2) (layer "F.Cu") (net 19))
 (segment (start 154.61515 21.03025) (end 149.85265 25.79275) (width 0.2) (layer "F.Cu") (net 19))
 (segment (start 176.42 25.98625) (end 176.6135 25.79275) (width 0.2) (layer "F.Cu") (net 19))
 (segment (start 130.56775 30.3965) (end 133.19125 33.02) (width 0.2) (layer "F.Cu") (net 19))
 (segment (start 176.6135 21.26515) (end 176.3786 21.03025) (width 0.2) (layer "F.Cu") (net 19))
 (segment (start 149.85265 25.79275) (end 130.80265 25.79275) (width 0.2) (layer "F.Cu") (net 19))
 (segment (start 130.56775 26.02765) (end 130.56775 30.3965) (width 0.2) (layer "F.Cu") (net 19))
 (segment (start 172.72 24.93125) (end 173.775 25.98625) (width 0.2) (layer "F.Cu") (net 19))
 (segment (start 173.775 25.98625) (end 176.42 25.98625) (width 0.2) (layer "F.Cu") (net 19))
 (segment (start 130.63655 25.39175) (end 130.16675 25.86155) (width 0.2) (layer "F.Cu") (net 18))
 (segment (start 130.764575 31.160425) (end 130.764575 45.833325) (width 0.2) (layer "F.Cu") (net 18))
 (segment (start 130.16675 30.5626) (end 130.764575 31.160425) (width 0.2) (layer "F.Cu") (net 18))
 (segment (start 154.44905 20.62925) (end 149.68655 25.39175) (width 0.2) (layer "F.Cu") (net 18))
 (segment (start 169.096 26.38725) (end 176.5861 26.38725) (width 0.2) (layer "F.Cu") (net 18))
 (segment (start 178.59375 23.8125) (end 177.0145 22.23325) (width 0.2) (layer "F.Cu") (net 18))
 (segment (start 130.764575 45.833325) (end 133.19125 48.26) (width 0.2) (layer "F.Cu") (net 18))
 (segment (start 177.0145 22.23325) (end 177.0145 21.09905) (width 0.2) (layer "F.Cu") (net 18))
 (segment (start 177.0145 21.09905) (end 176.5447 20.62925) (width 0.2) (layer "F.Cu") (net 18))
 (segment (start 130.16675 25.86155) (end 130.16675 30.5626) (width 0.2) (layer "F.Cu") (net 18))
 (segment (start 149.68655 25.39175) (end 130.63655 25.39175) (width 0.2) (layer "F.Cu") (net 18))
 (segment (start 167.64 24.93125) (end 169.096 26.38725) (width 0.2) (layer "F.Cu") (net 18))
 (segment (start 176.5861 26.38725) (end 178.59375 24.3796) (width 0.2) (layer "F.Cu") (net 18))
 (segment (start 176.5447 20.62925) (end 154.44905 20.62925) (width 0.2) (layer "F.Cu") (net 18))
 (segment (start 178.59375 24.3796) (end 178.59375 23.8125) (width 0.2) (layer "F.Cu") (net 18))
 (segment (start 187.28525 42.029) (end 134.34225 42.029) (width 0.2) (layer "F.Cu") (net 26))
 (segment (start 211.93125 35.8775) (end 195.10375 35.8775) (width 0.2) (layer "F.Cu") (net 26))
 (segment (start 134.34225 42.029) (end 133.19125 43.18) (width 0.2) (layer "F.Cu") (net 26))
 (segment (start 195.10375 35.8775) (end 188.11875 42.8625) (width 0.2) (layer "F.Cu") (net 26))
 (segment (start 188.11875 42.8625) (end 187.28525 42.029) (width 0.2) (layer "F.Cu") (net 26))
 (segment (start 197.32625 38.4175) (end 191.41275 44.331) (width 0.2) (layer "F.Cu") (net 28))
 (segment (start 191.41275 44.331) (end 134.58025 44.331) (width 0.2) (layer "F.Cu") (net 28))
 (segment (start 211.93125 38.4175) (end 197.32625 38.4175) (width 0.2) (layer "F.Cu") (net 28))
 (segment (start 134.58025 44.331) (end 133.19125 45.72) (width 0.2) (layer "F.Cu") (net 28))
 (segment (start 134.34225 39.489) (end 133.19125 40.64) (width 0.2) (layer "F.Cu") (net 25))
 (segment (start 135.25449 36.711) (end 134.34225 37.62324) (width 0.2) (layer "F.Cu") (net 25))
 (segment (start 139.58151 33.3375) (end 136.20801 36.711) (width 0.2) (layer "F.Cu") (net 25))
 (segment (start 211.93125 33.3375) (end 139.58151 33.3375) (width 0.2) (layer "F.Cu") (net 25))
 (segment (start 134.34225 37.62324) (end 134.34225 39.489) (width 0.2) (layer "F.Cu") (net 25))
 (segment (start 136.20801 36.711) (end 135.25449 36.711) (width 0.2) (layer "F.Cu") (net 25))
 (segment (start 147.6375 60.16625) (end 135.73125 48.26) (width 0.2) (layer "B.Cu") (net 29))
 (segment (start 169.4 61.9125) (end 147.6375 61.9125) (width 0.2) (layer "B.Cu") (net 29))
 (segment (start 173.29375 65.80625) (end 169.4 61.9125) (width 0.2) (layer "B.Cu") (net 29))
 (segment (start 147.6375 61.9125) (end 147.6375 60.16625) (width 0.2) (layer "B.Cu") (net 29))
 (segment (start 174.56875 59.53125) (end 149.5425 59.53125) (width 0.2) (layer "B.Cu") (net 1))
 (segment (start 180.84375 65.80625) (end 174.56875 59.53125) (width 0.2) (layer "B.Cu") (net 1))
 (segment (start 149.5425 59.53125) (end 135.73125 45.72) (width 0.2) (layer "B.Cu") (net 1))
 (segment (start 142.875 64.29375) (end 142.875 60.48375) (width 0.2) (layer "B.Cu") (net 5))
 (segment (start 142.875 60.48375) (end 135.73125 53.34) (width 0.2) (layer "B.Cu") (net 5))
 (segment (start 165.74375 65.80625) (end 164.23125 64.29375) (width 0.2) (layer "B.Cu") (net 5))
 (segment (start 164.23125 64.29375) (end 142.875 64.29375) (width 0.2) (layer "B.Cu") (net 5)))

